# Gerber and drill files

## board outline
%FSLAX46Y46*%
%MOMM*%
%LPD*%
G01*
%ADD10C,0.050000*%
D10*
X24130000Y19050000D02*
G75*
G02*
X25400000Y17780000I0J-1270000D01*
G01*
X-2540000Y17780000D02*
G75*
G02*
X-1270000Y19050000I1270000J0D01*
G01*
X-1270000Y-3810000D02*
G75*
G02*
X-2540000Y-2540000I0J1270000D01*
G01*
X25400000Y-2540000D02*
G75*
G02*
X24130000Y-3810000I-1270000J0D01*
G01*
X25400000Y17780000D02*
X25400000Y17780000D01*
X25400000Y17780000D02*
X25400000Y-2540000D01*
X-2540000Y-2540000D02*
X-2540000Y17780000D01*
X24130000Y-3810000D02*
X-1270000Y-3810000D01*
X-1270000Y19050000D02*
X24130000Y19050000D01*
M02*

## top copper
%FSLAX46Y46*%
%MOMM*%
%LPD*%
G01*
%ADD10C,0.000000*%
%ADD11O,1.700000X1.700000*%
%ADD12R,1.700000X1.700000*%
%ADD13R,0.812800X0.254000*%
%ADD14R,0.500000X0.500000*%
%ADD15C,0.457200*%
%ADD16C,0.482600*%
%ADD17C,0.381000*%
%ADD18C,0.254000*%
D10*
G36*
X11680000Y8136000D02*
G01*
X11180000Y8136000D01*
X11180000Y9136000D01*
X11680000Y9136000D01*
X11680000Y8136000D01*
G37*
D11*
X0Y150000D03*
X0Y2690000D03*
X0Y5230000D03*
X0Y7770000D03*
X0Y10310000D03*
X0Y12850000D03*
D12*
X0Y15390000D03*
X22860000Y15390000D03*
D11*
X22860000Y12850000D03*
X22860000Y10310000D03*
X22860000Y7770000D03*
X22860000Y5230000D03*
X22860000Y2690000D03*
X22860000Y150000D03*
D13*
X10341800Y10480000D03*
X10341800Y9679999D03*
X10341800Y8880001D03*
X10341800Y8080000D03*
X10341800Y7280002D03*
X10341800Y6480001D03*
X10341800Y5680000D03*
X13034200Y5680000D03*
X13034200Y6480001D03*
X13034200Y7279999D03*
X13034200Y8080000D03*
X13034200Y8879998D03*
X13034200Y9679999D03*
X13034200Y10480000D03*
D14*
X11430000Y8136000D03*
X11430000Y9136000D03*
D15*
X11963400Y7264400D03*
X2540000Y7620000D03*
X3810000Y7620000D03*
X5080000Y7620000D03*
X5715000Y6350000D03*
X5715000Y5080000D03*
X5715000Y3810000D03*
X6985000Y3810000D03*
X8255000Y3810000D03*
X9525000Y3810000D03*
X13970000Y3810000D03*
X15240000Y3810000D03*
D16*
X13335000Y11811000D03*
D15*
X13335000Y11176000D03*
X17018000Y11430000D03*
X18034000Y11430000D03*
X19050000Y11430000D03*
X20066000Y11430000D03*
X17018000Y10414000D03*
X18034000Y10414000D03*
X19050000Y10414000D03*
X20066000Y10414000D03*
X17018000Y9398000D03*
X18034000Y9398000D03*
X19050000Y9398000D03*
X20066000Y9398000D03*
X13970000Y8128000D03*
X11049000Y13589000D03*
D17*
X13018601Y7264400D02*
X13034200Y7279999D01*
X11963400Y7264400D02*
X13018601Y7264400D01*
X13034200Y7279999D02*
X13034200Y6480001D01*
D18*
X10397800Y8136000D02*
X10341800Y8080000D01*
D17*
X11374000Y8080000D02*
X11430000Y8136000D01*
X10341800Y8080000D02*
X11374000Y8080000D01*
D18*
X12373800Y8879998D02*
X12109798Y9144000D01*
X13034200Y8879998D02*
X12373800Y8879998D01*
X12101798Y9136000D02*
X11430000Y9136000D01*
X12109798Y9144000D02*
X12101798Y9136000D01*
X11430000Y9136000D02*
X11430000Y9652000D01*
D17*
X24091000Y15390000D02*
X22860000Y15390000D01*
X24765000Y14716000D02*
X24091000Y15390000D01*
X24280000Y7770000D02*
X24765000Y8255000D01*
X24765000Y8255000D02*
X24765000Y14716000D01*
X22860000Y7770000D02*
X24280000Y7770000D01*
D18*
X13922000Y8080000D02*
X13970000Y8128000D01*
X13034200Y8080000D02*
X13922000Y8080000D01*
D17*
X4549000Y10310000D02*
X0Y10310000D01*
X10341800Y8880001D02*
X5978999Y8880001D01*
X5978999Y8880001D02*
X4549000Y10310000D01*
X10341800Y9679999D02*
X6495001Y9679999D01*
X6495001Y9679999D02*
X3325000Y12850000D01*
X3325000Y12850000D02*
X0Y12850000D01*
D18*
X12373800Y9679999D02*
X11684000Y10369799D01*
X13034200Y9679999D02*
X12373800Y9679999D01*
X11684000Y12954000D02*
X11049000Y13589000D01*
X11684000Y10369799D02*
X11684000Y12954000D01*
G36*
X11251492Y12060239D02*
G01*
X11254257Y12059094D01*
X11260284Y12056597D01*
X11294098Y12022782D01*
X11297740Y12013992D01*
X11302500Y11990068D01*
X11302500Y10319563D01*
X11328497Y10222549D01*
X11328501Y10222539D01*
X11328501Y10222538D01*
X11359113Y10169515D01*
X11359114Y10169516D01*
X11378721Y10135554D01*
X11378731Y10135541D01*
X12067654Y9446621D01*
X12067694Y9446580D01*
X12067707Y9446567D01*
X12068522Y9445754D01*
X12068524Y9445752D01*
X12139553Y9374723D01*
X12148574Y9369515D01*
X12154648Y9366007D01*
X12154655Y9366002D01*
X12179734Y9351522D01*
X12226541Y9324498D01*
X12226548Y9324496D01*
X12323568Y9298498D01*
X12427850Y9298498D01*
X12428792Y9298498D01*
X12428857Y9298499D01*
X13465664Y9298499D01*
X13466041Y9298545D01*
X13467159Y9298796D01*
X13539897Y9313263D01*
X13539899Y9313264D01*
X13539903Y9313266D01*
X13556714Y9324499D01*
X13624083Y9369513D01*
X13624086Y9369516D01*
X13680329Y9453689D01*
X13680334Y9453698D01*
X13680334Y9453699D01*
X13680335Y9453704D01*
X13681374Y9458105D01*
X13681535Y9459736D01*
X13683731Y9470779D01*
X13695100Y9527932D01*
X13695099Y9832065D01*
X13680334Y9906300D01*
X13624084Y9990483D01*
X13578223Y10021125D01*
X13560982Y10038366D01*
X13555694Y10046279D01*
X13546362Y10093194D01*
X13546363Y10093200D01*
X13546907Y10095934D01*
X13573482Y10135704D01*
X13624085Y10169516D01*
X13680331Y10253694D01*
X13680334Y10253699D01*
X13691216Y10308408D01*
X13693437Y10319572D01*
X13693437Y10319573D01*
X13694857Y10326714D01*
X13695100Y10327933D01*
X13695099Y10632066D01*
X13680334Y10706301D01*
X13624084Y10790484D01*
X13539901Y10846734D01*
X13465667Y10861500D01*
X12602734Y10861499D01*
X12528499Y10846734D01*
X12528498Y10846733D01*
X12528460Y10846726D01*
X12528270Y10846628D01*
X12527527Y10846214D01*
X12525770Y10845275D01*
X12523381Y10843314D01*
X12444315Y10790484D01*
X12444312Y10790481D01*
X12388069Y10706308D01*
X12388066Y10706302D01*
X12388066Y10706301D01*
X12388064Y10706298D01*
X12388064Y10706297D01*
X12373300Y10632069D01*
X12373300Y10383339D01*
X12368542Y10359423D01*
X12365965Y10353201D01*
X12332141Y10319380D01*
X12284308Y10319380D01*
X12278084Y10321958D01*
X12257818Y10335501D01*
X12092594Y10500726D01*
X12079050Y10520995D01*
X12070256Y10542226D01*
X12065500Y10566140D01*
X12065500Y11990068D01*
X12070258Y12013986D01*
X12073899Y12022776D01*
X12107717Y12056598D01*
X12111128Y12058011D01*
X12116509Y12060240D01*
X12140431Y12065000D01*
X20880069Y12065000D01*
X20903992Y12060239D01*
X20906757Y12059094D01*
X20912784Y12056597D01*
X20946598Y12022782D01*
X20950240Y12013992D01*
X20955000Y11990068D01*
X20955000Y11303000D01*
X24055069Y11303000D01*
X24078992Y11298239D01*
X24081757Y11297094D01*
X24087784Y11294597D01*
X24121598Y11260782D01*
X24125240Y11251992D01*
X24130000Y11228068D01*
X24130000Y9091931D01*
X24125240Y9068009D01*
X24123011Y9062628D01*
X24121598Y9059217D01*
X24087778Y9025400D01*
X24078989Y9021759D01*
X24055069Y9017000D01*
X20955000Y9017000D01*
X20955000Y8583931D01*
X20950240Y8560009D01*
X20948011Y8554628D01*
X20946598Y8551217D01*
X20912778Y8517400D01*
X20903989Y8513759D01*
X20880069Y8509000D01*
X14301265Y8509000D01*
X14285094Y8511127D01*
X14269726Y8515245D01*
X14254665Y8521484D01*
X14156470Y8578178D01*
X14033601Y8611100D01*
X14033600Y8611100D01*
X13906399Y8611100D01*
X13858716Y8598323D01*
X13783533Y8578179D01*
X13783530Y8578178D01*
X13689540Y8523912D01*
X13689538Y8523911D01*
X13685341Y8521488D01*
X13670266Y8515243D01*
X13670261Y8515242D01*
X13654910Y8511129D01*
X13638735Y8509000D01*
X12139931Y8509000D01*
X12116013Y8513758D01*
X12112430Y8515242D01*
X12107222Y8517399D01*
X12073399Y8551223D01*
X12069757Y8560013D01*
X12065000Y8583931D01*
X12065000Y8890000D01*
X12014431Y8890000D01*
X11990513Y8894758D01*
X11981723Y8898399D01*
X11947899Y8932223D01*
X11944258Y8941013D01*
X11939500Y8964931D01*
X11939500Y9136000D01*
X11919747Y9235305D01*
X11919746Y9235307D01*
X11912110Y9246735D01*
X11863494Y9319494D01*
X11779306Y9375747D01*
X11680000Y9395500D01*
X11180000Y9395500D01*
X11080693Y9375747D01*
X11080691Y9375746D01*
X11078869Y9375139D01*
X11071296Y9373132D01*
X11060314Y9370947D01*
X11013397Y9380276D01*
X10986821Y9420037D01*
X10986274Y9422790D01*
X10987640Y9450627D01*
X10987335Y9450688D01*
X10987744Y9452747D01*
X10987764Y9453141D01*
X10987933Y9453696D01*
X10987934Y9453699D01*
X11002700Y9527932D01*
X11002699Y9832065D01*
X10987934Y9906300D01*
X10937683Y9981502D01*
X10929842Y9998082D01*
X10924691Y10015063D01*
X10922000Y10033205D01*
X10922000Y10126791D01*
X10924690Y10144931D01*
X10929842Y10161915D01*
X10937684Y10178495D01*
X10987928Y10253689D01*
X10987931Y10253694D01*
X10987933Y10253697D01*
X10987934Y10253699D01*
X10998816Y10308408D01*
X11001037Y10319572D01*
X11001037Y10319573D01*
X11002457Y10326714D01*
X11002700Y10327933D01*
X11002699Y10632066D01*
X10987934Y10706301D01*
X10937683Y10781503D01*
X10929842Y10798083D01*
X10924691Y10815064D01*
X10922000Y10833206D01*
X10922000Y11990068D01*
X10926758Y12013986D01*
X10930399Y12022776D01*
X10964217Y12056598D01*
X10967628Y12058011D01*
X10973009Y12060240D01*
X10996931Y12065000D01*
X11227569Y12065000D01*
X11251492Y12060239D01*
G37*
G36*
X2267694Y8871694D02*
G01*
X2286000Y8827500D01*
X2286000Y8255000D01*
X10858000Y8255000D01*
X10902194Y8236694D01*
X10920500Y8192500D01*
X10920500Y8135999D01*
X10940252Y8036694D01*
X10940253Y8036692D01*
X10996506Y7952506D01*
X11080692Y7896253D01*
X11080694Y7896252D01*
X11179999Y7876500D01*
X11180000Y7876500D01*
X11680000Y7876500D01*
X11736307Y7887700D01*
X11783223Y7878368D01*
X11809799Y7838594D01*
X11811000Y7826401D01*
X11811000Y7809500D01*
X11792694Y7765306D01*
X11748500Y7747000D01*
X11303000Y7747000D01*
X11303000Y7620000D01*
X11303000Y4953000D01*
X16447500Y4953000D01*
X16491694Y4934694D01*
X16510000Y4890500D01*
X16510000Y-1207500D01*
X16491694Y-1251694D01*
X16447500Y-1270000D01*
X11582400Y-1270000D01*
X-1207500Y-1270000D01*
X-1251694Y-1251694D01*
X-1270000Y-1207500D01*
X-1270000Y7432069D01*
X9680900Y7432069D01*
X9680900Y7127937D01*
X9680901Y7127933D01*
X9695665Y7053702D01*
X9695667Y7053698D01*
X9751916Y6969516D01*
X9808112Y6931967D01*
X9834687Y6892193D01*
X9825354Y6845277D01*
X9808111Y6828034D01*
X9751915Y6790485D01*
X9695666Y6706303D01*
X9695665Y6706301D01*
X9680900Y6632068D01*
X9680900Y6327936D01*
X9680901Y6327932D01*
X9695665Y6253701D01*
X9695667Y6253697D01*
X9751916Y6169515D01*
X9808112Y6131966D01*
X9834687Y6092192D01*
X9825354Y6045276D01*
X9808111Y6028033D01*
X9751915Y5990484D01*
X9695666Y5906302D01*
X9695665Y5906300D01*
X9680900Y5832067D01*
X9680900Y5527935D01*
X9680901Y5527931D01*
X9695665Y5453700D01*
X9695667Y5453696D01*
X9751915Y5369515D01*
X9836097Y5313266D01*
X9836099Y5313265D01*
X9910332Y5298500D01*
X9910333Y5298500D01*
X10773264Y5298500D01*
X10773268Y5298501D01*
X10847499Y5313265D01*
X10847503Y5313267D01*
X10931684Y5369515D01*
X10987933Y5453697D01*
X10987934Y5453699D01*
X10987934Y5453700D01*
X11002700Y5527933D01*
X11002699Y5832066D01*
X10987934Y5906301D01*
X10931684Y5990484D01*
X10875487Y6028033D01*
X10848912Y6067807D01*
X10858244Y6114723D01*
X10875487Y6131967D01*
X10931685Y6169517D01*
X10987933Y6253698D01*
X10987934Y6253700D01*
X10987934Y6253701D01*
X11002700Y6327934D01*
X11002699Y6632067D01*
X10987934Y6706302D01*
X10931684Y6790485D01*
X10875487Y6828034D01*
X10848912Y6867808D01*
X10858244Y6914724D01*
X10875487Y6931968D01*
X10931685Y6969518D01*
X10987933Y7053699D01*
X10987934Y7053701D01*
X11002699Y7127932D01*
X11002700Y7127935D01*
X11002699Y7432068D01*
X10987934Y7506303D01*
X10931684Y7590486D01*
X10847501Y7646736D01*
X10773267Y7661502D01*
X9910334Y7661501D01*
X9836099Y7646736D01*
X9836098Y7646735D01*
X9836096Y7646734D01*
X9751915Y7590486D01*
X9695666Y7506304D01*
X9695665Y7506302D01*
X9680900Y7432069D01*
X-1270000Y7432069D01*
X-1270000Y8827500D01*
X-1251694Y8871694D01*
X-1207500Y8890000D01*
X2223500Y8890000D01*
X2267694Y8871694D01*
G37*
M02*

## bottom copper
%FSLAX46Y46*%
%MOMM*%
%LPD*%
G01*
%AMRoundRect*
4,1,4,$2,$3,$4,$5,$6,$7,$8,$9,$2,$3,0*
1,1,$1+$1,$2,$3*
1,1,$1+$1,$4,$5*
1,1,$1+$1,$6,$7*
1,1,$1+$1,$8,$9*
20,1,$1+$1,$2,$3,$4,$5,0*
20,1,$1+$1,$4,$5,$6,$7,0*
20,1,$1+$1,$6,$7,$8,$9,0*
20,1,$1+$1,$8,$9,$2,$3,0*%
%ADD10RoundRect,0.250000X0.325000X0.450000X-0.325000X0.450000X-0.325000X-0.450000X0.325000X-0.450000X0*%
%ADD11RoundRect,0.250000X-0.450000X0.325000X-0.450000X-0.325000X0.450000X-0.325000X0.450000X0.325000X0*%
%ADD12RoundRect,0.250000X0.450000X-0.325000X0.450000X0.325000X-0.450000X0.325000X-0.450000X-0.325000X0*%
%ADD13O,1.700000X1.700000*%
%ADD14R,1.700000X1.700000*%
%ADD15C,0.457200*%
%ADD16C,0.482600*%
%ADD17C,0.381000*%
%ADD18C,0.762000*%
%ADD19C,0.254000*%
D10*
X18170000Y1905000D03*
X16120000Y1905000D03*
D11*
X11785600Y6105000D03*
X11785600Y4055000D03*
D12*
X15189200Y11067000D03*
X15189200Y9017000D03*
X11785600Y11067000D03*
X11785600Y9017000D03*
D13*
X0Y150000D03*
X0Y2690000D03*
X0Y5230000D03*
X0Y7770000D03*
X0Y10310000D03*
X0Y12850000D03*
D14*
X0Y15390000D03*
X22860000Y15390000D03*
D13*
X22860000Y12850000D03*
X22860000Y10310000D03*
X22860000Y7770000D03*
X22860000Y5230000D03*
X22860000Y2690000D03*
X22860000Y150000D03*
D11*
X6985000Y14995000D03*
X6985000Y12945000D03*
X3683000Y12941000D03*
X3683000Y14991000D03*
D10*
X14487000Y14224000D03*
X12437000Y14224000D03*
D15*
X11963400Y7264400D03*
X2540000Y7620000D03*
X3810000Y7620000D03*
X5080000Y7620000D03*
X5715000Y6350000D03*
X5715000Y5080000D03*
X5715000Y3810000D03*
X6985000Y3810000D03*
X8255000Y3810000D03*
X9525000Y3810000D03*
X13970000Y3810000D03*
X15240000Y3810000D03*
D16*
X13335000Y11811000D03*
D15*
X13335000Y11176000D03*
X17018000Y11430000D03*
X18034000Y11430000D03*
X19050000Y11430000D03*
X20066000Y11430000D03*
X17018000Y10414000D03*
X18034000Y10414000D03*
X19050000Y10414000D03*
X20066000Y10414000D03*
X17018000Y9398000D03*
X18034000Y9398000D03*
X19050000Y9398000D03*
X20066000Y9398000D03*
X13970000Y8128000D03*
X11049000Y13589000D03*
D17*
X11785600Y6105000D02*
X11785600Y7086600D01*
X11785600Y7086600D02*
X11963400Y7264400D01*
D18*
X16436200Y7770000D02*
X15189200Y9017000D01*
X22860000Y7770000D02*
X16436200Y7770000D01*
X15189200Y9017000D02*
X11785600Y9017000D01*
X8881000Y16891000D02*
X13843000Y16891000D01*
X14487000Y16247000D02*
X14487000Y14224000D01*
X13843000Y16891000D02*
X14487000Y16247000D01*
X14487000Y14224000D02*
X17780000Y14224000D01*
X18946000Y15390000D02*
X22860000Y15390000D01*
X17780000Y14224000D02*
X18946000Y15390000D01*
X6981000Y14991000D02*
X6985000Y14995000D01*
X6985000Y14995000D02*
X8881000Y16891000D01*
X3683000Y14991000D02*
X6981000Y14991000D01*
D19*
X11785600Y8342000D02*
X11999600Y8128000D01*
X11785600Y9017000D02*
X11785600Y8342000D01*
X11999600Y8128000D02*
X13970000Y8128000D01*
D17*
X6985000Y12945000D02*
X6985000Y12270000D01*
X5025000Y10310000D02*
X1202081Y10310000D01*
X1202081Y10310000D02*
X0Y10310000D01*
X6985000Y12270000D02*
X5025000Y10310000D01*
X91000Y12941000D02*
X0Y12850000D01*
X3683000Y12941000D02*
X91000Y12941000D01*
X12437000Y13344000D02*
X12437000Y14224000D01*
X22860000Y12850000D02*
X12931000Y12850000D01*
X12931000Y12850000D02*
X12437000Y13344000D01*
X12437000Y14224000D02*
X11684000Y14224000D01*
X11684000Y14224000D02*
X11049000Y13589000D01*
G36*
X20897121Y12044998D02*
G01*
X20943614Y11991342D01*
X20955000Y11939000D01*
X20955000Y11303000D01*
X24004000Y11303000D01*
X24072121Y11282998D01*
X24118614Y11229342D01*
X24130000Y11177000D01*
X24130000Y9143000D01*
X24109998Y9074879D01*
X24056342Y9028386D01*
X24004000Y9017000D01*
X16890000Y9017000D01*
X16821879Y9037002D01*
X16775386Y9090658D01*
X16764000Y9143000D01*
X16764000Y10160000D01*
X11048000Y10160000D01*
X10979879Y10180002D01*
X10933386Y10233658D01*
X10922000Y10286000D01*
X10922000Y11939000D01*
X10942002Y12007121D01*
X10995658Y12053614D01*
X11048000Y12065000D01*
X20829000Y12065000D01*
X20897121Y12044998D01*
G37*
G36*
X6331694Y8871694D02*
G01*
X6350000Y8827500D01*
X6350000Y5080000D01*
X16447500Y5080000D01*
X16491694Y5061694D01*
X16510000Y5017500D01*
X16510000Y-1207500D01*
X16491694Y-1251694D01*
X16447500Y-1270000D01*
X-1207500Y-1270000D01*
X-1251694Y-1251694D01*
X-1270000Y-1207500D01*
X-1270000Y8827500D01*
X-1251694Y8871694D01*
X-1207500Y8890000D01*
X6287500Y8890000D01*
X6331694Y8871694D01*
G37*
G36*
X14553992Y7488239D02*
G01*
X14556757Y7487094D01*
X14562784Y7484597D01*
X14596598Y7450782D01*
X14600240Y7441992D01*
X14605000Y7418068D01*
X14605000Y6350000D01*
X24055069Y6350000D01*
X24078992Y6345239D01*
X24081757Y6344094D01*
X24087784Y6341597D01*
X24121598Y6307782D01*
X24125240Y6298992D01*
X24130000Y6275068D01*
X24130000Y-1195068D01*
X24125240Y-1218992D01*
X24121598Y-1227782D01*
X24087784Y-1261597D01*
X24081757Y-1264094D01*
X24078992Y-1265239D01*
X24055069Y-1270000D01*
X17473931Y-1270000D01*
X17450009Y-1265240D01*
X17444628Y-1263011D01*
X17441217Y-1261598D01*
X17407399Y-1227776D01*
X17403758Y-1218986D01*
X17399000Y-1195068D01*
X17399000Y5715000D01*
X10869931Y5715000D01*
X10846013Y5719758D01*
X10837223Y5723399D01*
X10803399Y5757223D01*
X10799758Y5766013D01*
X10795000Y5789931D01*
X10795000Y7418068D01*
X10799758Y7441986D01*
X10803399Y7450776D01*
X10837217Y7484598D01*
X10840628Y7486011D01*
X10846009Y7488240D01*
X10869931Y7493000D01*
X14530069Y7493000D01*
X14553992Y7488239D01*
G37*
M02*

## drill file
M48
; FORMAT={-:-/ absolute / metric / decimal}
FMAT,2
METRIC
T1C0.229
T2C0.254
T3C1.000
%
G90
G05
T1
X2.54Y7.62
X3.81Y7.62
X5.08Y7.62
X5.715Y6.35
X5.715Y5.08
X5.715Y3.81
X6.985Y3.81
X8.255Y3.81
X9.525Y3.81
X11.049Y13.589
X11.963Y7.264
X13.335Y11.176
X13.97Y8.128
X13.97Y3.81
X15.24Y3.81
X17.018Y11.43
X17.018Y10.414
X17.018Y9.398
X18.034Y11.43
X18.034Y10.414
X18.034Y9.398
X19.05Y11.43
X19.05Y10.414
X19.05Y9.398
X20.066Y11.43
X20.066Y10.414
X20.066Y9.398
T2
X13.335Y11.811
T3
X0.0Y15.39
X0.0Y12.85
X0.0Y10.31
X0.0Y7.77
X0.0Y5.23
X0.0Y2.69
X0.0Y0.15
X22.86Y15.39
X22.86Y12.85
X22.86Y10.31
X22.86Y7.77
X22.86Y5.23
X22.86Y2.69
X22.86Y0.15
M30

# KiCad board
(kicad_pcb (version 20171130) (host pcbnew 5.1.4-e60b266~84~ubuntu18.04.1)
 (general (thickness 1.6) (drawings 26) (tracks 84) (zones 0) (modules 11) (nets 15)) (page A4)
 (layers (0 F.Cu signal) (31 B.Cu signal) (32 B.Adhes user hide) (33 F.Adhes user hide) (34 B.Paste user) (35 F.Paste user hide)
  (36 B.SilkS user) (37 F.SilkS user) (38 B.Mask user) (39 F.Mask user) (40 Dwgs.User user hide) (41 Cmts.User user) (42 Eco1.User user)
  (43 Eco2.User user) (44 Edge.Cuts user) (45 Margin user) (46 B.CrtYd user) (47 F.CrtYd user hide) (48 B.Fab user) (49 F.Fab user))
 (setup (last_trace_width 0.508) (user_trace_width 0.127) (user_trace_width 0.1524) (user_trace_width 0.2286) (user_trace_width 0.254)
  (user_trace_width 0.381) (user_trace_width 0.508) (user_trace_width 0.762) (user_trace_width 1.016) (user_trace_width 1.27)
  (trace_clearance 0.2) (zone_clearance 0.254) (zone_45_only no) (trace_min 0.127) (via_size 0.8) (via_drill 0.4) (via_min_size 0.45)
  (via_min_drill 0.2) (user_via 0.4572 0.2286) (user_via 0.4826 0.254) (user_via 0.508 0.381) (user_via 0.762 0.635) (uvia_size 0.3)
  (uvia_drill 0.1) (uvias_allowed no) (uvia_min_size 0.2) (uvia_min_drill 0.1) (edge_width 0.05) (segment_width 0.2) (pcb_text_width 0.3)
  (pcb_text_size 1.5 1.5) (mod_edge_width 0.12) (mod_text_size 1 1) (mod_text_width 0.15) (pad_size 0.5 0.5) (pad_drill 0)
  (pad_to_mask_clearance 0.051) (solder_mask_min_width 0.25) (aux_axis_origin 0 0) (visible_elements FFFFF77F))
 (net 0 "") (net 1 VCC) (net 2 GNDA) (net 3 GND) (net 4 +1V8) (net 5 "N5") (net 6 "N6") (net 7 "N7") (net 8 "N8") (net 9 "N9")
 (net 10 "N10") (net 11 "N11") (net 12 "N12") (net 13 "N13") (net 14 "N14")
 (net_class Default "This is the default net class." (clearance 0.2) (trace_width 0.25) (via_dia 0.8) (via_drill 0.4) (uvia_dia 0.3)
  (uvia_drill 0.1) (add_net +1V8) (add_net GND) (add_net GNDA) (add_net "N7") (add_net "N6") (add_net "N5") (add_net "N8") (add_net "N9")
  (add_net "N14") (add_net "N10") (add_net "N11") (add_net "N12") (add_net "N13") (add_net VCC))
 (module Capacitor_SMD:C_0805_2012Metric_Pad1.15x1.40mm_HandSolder (layer B.Cu) (at 17.145 -1.905 180)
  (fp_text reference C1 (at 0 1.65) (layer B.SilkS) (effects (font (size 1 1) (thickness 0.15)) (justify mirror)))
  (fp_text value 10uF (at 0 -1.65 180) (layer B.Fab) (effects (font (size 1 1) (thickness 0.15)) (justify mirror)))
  (pad 1 smd roundrect (at -1.025 0 180) (size 1.15 1.4) (layers B.Cu B.Paste B.Mask) (roundrect_rratio 0.217391) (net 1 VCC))
  (pad 2 smd roundrect (at 1.025 0 180) (size 1.15 1.4) (layers B.Cu B.Paste B.Mask) (roundrect_rratio 0.217391) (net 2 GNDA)))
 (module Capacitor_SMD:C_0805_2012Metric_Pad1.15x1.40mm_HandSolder (layer B.Cu) (at 11.7856 -5.08 270)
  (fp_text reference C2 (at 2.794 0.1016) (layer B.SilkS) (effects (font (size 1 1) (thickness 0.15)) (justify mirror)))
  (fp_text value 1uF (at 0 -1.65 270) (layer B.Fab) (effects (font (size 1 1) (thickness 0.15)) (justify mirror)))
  (pad 1 smd roundrect (at -1.025 0 270) (size 1.15 1.4) (layers B.Cu B.Paste B.Mask) (roundrect_rratio 0.217391) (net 1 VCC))
  (pad 2 smd roundrect (at 1.025 0 270) (size 1.15 1.4) (layers B.Cu B.Paste B.Mask) (roundrect_rratio 0.217391) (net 2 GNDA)))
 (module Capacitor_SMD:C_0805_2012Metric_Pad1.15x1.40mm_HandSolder (layer B.Cu) (at 15.1892 -10.042 90)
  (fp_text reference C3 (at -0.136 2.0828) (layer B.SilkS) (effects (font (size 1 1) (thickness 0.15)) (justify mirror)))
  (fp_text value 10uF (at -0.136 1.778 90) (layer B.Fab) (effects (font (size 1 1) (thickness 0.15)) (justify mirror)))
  (pad 2 smd roundrect (at 1.025 0 90) (size 1.15 1.4) (layers B.Cu B.Paste B.Mask) (roundrect_rratio 0.217391) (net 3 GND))
  (pad 1 smd roundrect (at -1.025 0 90) (size 1.15 1.4) (layers B.Cu B.Paste B.Mask) (roundrect_rratio 0.217391) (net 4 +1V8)))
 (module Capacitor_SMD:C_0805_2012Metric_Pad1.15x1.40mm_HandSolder (layer B.Cu) (at 11.7856 -10.042 90)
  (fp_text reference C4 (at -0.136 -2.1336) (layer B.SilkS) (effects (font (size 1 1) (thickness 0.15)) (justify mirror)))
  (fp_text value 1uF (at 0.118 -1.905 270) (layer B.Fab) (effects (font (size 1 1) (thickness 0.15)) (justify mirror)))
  (pad 2 smd roundrect (at 1.025 0 90) (size 1.15 1.4) (layers B.Cu B.Paste B.Mask) (roundrect_rratio 0.217391) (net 3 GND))
  (pad 1 smd roundrect (at -1.025 0 90) (size 1.15 1.4) (layers B.Cu B.Paste B.Mask) (roundrect_rratio 0.217391) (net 4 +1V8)))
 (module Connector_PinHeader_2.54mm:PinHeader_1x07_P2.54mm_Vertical (layer F.Cu) (at 0 -15.39)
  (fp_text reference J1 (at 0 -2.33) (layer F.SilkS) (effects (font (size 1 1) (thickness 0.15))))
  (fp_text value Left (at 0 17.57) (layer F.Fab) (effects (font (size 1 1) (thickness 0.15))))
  (pad 7 thru_hole oval (at 0 15.24) (size 1.7 1.7) (drill 1) (layers *.Cu *.Mask) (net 2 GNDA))
  (pad 6 thru_hole oval (at 0 12.7) (size 1.7 1.7) (drill 1) (layers *.Cu *.Mask) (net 2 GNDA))
  (pad 5 thru_hole oval (at 0 10.16) (size 1.7 1.7) (drill 1) (layers *.Cu *.Mask) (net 2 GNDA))
  (pad 4 thru_hole oval (at 0 7.62) (size 1.7 1.7) (drill 1) (layers *.Cu *.Mask) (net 2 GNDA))
  (pad 3 thru_hole oval (at 0 5.08) (size 1.7 1.7) (drill 1) (layers *.Cu *.Mask) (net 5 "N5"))
  (pad 2 thru_hole oval (at 0 2.54) (size 1.7 1.7) (drill 1) (layers *.Cu *.Mask) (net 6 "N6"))
  (pad 1 thru_hole rect (at 0 0) (size 1.7 1.7) (drill 1) (layers *.Cu *.Mask) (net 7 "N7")))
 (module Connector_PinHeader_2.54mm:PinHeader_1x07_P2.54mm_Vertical (layer F.Cu) (at 22.86 -15.39)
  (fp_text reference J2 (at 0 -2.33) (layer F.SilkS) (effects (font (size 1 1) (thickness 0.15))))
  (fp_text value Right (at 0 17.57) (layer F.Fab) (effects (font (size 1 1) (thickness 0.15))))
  (pad 1 thru_hole rect (at 0 0) (size 1.7 1.7) (drill 1) (layers *.Cu *.Mask) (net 4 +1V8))
  (pad 2 thru_hole oval (at 0 2.54) (size 1.7 1.7) (drill 1) (layers *.Cu *.Mask) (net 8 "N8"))
  (pad 3 thru_hole oval (at 0 5.08) (size 1.7 1.7) (drill 1) (layers *.Cu *.Mask) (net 3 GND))
  (pad 4 thru_hole oval (at 0 7.62) (size 1.7 1.7) (drill 1) (layers *.Cu *.Mask) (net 4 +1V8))
  (pad 5 thru_hole oval (at 0 10.16) (size 1.7 1.7) (drill 1) (layers *.Cu *.Mask) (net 1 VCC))
  (pad 6 thru_hole oval (at 0 12.7) (size 1.7 1.7) (drill 1) (layers *.Cu *.Mask) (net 1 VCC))
  (pad 7 thru_hole oval (at 0 15.24) (size 1.7 1.7) (drill 1) (layers *.Cu *.Mask) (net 1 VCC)))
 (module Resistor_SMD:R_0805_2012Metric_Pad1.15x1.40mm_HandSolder (layer B.Cu) (at 6.985 -13.97 270)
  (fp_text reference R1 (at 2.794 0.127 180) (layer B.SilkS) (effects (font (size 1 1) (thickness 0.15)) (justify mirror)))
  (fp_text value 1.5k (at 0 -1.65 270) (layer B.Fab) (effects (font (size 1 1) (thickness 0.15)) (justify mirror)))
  (pad 1 smd roundrect (at -1.025 0 270) (size 1.15 1.4) (layers B.Cu B.Paste B.Mask) (roundrect_rratio 0.217391) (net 4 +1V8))
  (pad 2 smd roundrect (at 1.025 0 270) (size 1.15 1.4) (layers B.Cu B.Paste B.Mask) (roundrect_rratio 0.217391) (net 5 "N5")))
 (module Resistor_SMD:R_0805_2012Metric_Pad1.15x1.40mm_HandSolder (layer B.Cu) (at 3.683 -13.966 270)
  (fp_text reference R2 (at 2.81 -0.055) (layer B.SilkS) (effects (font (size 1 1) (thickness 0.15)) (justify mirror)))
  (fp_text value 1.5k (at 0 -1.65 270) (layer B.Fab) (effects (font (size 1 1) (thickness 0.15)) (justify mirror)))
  (pad 2 smd roundrect (at 1.025 0 270) (size 1.15 1.4) (layers B.Cu B.Paste B.Mask) (roundrect_rratio 0.217391) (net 6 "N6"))
  (pad 1 smd roundrect (at -1.025 0 270) (size 1.15 1.4) (layers B.Cu B.Paste B.Mask) (roundrect_rratio 0.217391) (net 4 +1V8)))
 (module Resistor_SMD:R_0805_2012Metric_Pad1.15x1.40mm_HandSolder (layer B.Cu) (at 13.462 -14.224 180)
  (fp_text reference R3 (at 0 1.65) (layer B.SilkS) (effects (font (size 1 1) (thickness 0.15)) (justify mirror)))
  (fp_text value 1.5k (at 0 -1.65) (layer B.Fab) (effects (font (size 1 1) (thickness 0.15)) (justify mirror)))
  (pad 1 smd roundrect (at -1.025 0 180) (size 1.15 1.4) (layers B.Cu B.Paste B.Mask) (roundrect_rratio 0.217391) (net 4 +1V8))
  (pad 2 smd roundrect (at 1.025 0 180) (size 1.15 1.4) (layers B.Cu B.Paste B.Mask) (roundrect_rratio 0.217391) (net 8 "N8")))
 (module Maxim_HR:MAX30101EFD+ (layer F.Cu) (at 11.688 -8.08)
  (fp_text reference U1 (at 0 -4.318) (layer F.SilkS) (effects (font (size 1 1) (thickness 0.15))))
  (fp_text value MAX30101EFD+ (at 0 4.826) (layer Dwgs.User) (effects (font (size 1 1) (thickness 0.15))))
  (pad 1 smd rect (at -1.3462 -2.4) (size 0.8128 0.254) (layers F.Cu F.Paste F.Mask) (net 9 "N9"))
  (pad 2 smd rect (at -1.3462 -1.599999) (size 0.8128 0.254) (layers F.Cu F.Paste F.Mask) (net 6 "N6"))
  (pad 3 smd rect (at -1.3462 -0.800001) (size 0.8128 0.254) (layers F.Cu F.Paste F.Mask) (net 5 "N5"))
  (pad 4 smd rect (at -1.3462 0) (size 0.8128 0.254) (layers F.Cu F.Paste F.Mask) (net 2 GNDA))
  (pad 5 smd rect (at -1.3462 0.799998) (size 0.8128 0.254) (layers F.Cu F.Paste F.Mask) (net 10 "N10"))
  (pad 6 smd rect (at -1.3462 1.599999) (size 0.8128 0.254) (layers F.Cu F.Paste F.Mask) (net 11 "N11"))
  (pad 7 smd rect (at -1.3462 2.4) (size 0.8128 0.254) (layers F.Cu F.Paste F.Mask) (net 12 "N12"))
  (pad 8 smd rect (at 1.3462 2.4) (size 0.8128 0.254) (layers F.Cu F.Paste F.Mask) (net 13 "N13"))
  (pad 9 smd rect (at 1.3462 1.599999) (size 0.8128 0.254) (layers F.Cu F.Paste F.Mask) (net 1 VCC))
  (pad 10 smd rect (at 1.3462 0.800001) (size 0.8128 0.254) (layers F.Cu F.Paste F.Mask) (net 1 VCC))
  (pad 11 smd rect (at 1.3462 0) (size 0.8128 0.254) (layers F.Cu F.Paste F.Mask) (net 4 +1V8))
  (pad 12 smd rect (at 1.3462 -0.799998) (size 0.8128 0.254) (layers F.Cu F.Paste F.Mask) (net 3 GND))
  (pad 13 smd rect (at 1.3462 -1.599999) (size 0.8128 0.254) (layers F.Cu F.Paste F.Mask) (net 8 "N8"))
  (pad 14 smd rect (at 1.3462 -2.4) (size 0.8128 0.254) (layers F.Cu F.Paste F.Mask) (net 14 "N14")))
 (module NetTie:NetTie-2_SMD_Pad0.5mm (layer F.Cu) (at 11.43 -8.636 90)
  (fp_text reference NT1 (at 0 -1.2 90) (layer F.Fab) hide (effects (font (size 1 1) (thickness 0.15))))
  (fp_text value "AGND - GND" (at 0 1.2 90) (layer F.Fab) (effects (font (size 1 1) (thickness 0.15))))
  (fp_poly (pts (xy -0.5 -0.25) (xy 0.5 -0.25) (xy 0.5 0.25) (xy -0.5 0.25)) (layer F.Cu) (width 0))
  (pad 1 smd rect (at -0.5 0 90) (size 0.5 0.5) (layers F.Cu) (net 2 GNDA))
  (pad 2 smd rect (at 0.5 0 90) (size 0.5 0.5) (layers F.Cu) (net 3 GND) (zone_connect 2) (thermal_width 1.27) (thermal_gap 0.127)))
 (gr_arc (start 24.13 -17.78) (end 25.4 -17.78) (angle -90) (layer Edge.Cuts) (width 0.05))
 (gr_arc (start -1.27 -17.78) (end -1.27 -19.05) (angle -90) (layer Edge.Cuts) (width 0.05))
 (gr_arc (start -1.27 2.54) (end -2.54 2.54) (angle -90) (layer Edge.Cuts) (width 0.05))
 (gr_arc (start 24.13 2.54) (end 24.13 3.81) (angle -90) (layer Edge.Cuts) (width 0.05))
 (gr_line (start 25.4 -17.78) (end 25.4 -17.78) (layer Edge.Cuts) (width 0.05))
 (gr_line (start 25.4 -17.78) (end 25.4 2.54) (layer Edge.Cuts) (width 0.05))
 (gr_line (start -2.54 2.54) (end -2.54 -17.78) (layer Edge.Cuts) (width 0.05))
 (gr_line (start 24.13 3.81) (end -1.27 3.81) (layer Edge.Cuts) (width 0.05))
 (gr_line (start -1.27 -19.05) (end 24.13 -19.05) (layer Edge.Cuts) (width 0.05))
 (via (at 11.9634 -7.2644) (size 0.4572) (drill 0.2286) (layers F.Cu B.Cu) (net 1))
 (segment (start 11.7856 -6.105) (end 11.7856 -7.0866) (width 0.381) (layer B.Cu) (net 1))
 (segment (start 11.7856 -7.0866) (end 11.9634 -7.2644) (width 0.381) (layer B.Cu) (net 1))
 (segment (start 13.018601 -7.2644) (end 13.0342 -7.279999) (width 0.381) (layer F.Cu) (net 1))
 (segment (start 11.9634 -7.2644) (end 13.018601 -7.2644) (width 0.381) (layer F.Cu) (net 1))
 (segment (start 13.0342 -7.279999) (end 13.0342 -6.480001) (width 0.381) (layer F.Cu) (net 1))
 (segment (start 10.3978 -8.136) (end 10.3418 -8.08) (width 0.254) (layer F.Cu) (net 2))
 (via (at 2.54 -7.62) (size 0.4572) (drill 0.2286) (layers F.Cu B.Cu) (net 2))
 (via (at 3.81 -7.62) (size 0.4572) (drill 0.2286) (layers F.Cu B.Cu) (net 2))
 (via (at 5.08 -7.62) (size 0.4572) (drill 0.2286) (layers F.Cu B.Cu) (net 2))
 (via (at 5.715 -6.35) (size 0.4572) (drill 0.2286) (layers F.Cu B.Cu) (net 2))
 (via (at 5.715 -5.08) (size 0.4572) (drill 0.2286) (layers F.Cu B.Cu) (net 2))
 (via (at 5.715 -3.81) (size 0.4572) (drill 0.2286) (layers F.Cu B.Cu) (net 2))
 (via (at 6.985 -3.81) (size 0.4572) (drill 0.2286) (layers F.Cu B.Cu) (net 2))
 (via (at 8.255 -3.81) (size 0.4572) (drill 0.2286) (layers F.Cu B.Cu) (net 2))
 (via (at 9.525 -3.81) (size 0.4572) (drill 0.2286) (layers F.Cu B.Cu) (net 2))
 (via (at 13.97 -3.81) (size 0.4572) (drill 0.2286) (layers F.Cu B.Cu) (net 2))
 (via (at 15.24 -3.81) (size 0.4572) (drill 0.2286) (layers F.Cu B.Cu) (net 2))
 (segment (start 11.374 -8.08) (end 11.43 -8.136) (width 0.381) (layer F.Cu) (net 2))
 (segment (start 10.3418 -8.08) (end 11.374 -8.08) (width 0.381) (layer F.Cu) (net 2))
 (via (at 13.335 -11.811) (size 0.4826) (drill 0.254) (layers F.Cu B.Cu) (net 3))
 (via (at 13.335 -11.176) (size 0.4572) (drill 0.2286) (layers F.Cu B.Cu) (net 3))
 (segment (start 12.3738 -8.879998) (end 12.109798 -9.144) (width 0.254) (layer F.Cu) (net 3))
 (segment (start 13.0342 -8.879998) (end 12.3738 -8.879998) (width 0.254) (layer F.Cu) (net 3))
 (segment (start 12.101798 -9.136) (end 11.43 -9.136) (width 0.254) (layer F.Cu) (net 3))
 (segment (start 12.109798 -9.144) (end 12.101798 -9.136) (width 0.254) (layer F.Cu) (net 3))
 (segment (start 11.43 -9.136) (end 11.43 -9.652) (width 0.254) (layer F.Cu) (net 3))
 (via (at 17.018 -11.43) (size 0.4572) (drill 0.2286) (layers F.Cu B.Cu) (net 3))
 (via (at 18.034 -11.43) (size 0.4572) (drill 0.2286) (layers F.Cu B.Cu) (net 3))
 (via (at 19.05 -11.43) (size 0.4572) (drill 0.2286) (layers F.Cu B.Cu) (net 3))
 (via (at 20.066 -11.43) (size 0.4572) (drill 0.2286) (layers F.Cu B.Cu) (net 3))
 (via (at 17.018 -10.414) (size 0.4572) (drill 0.2286) (layers F.Cu B.Cu) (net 3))
 (via (at 18.034 -10.414) (size 0.4572) (drill 0.2286) (layers F.Cu B.Cu) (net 3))
 (via (at 19.05 -10.414) (size 0.4572) (drill 0.2286) (layers F.Cu B.Cu) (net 3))
 (via (at 20.066 -10.414) (size 0.4572) (drill 0.2286) (layers F.Cu B.Cu) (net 3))
 (via (at 17.018 -9.398) (size 0.4572) (drill 0.2286) (layers F.Cu B.Cu) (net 3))
 (via (at 18.034 -9.398) (size 0.4572) (drill 0.2286) (layers F.Cu B.Cu) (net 3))
 (via (at 19.05 -9.398) (size 0.4572) (drill 0.2286) (layers F.Cu B.Cu) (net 3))
 (via (at 20.066 -9.398) (size 0.4572) (drill 0.2286) (layers F.Cu B.Cu) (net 3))
 (segment (start 16.4362 -7.77) (end 15.1892 -9.017) (width 0.762) (layer B.Cu) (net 4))
 (segment (start 22.86 -7.77) (end 16.4362 -7.77) (width 0.762) (layer B.Cu) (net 4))
 (segment (start 15.1892 -9.017) (end 11.7856 -9.017) (width 0.762) (layer B.Cu) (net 4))
 (segment (start 8.881 -16.891) (end 13.843 -16.891) (width 0.762) (layer B.Cu) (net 4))
 (segment (start 14.487 -16.247) (end 14.487 -14.224) (width 0.762) (layer B.Cu) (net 4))
 (segment (start 13.843 -16.891) (end 14.487 -16.247) (width 0.762) (layer B.Cu) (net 4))
 (segment (start 14.487 -14.224) (end 17.78 -14.224) (width 0.762) (layer B.Cu) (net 4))
 (segment (start 18.946 -15.39) (end 22.86 -15.39) (width 0.762) (layer B.Cu) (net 4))
 (segment (start 17.78 -14.224) (end 18.946 -15.39) (width 0.762) (layer B.Cu) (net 4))
 (segment (start 6.981 -14.991) (end 6.985 -14.995) (width 0.762) (layer B.Cu) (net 4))
 (segment (start 6.985 -14.995) (end 8.881 -16.891) (width 0.762) (layer B.Cu) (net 4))
 (segment (start 3.683 -14.991) (end 6.981 -14.991) (width 0.762) (layer B.Cu) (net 4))
 (segment (start 24.091 -15.39) (end 22.86 -15.39) (width 0.381) (layer F.Cu) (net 4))
 (segment (start 24.765 -14.716) (end 24.091 -15.39) (width 0.381) (layer F.Cu) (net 4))
 (segment (start 24.28 -7.77) (end 24.765 -8.255) (width 0.381) (layer F.Cu) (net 4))
 (segment (start 24.765 -8.255) (end 24.765 -14.716) (width 0.381) (layer F.Cu) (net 4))
 (segment (start 22.86 -7.77) (end 24.28 -7.77) (width 0.381) (layer F.Cu) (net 4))
 (segment (start 11.7856 -8.342) (end 11.9996 -8.128) (width 0.254) (layer B.Cu) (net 4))
 (segment (start 11.7856 -9.017) (end 11.7856 -8.342) (width 0.254) (layer B.Cu) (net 4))
 (via (at 13.97 -8.128) (size 0.4572) (drill 0.2286) (layers F.Cu B.Cu) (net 4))
 (segment (start 11.9996 -8.128) (end 13.97 -8.128) (width 0.254) (layer B.Cu) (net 4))
 (segment (start 13.922 -8.08) (end 13.97 -8.128) (width 0.254) (layer F.Cu) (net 4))
 (segment (start 13.0342 -8.08) (end 13.922 -8.08) (width 0.254) (layer F.Cu) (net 4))
 (segment (start 4.549 -10.31) (end 0 -10.31) (width 0.381) (layer F.Cu) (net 5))
 (segment (start 10.3418 -8.880001) (end 5.978999 -8.880001) (width 0.381) (layer F.Cu) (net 5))
 (segment (start 5.978999 -8.880001) (end 4.549 -10.31) (width 0.381) (layer F.Cu) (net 5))
 (segment (start 6.985 -12.945) (end 6.985 -12.27) (width 0.381) (layer B.Cu) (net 5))
 (segment (start 5.025 -10.31) (end 1.202081 -10.31) (width 0.381) (layer B.Cu) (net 5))
 (segment (start 1.202081 -10.31) (end 0 -10.31) (width 0.381) (layer B.Cu) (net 5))
 (segment (start 6.985 -12.27) (end 5.025 -10.31) (width 0.381) (layer B.Cu) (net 5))
 (segment (start 10.3418 -9.679999) (end 6.495001 -9.679999) (width 0.381) (layer F.Cu) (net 6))
 (segment (start 6.495001 -9.679999) (end 3.325 -12.85) (width 0.381) (layer F.Cu) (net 6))
 (segment (start 3.325 -12.85) (end 0 -12.85) (width 0.381) (layer F.Cu) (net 6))
 (segment (start 0.091 -12.941) (end 0 -12.85) (width 0.381) (layer B.Cu) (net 6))
 (segment (start 3.683 -12.941) (end 0.091 -12.941) (width 0.381) (layer B.Cu) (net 6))
 (segment (start 12.437 -13.344) (end 12.437 -14.224) (width 0.381) (layer B.Cu) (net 8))
 (segment (start 22.86 -12.85) (end 12.931 -12.85) (width 0.381) (layer B.Cu) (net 8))
 (segment (start 12.931 -12.85) (end 12.437 -13.344) (width 0.381) (layer B.Cu) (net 8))
 (via (at 11.049 -13.589) (size 0.4572) (drill 0.2286) (layers F.Cu B.Cu) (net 8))
 (segment (start 12.437 -14.224) (end 11.684 -14.224) (width 0.381) (layer B.Cu) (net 8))
 (segment (start 11.684 -14.224) (end 11.049 -13.589) (width 0.381) (layer B.Cu) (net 8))
 (segment (start 12.3738 -9.679999) (end 11.684 -10.369799) (width 0.254) (layer F.Cu) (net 8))
 (segment (start 13.0342 -9.679999) (end 12.3738 -9.679999) (width 0.254) (layer F.Cu) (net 8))
 (segment (start 11.684 -12.954) (end 11.049 -13.589) (width 0.254) (layer F.Cu) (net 8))
 (segment (start 11.684 -10.369799) (end 11.684 -12.954) (width 0.254) (layer F.Cu) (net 8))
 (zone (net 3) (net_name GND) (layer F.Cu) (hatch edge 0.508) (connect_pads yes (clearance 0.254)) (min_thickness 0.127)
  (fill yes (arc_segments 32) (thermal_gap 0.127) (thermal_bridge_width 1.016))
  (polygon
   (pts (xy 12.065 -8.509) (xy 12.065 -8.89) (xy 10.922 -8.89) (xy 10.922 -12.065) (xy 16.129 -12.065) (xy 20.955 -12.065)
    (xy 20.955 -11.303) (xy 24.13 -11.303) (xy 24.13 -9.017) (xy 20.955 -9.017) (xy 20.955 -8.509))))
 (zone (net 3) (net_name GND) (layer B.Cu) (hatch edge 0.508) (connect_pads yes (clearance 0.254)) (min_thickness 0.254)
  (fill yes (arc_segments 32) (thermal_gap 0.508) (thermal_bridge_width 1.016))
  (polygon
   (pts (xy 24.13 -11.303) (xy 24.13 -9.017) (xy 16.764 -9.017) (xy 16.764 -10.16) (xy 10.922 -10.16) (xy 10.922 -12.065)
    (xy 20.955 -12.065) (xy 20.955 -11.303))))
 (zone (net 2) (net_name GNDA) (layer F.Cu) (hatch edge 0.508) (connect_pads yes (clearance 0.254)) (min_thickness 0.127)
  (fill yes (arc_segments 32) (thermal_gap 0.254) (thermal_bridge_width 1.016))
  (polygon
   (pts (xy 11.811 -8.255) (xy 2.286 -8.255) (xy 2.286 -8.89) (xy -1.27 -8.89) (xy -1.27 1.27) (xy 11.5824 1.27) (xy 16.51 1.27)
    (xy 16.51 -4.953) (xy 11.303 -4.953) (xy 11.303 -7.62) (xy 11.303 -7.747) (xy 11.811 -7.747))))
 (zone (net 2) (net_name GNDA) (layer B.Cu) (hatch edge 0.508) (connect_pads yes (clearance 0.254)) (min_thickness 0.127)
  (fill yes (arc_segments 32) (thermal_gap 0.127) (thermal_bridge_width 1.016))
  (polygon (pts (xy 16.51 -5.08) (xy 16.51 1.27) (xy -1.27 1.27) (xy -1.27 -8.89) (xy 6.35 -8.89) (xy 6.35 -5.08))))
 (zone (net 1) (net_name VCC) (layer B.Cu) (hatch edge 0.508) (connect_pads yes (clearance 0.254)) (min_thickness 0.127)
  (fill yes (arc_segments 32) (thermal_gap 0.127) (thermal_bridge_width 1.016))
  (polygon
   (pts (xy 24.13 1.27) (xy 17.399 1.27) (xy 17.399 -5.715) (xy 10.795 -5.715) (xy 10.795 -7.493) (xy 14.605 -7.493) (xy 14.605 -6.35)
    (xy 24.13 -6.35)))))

